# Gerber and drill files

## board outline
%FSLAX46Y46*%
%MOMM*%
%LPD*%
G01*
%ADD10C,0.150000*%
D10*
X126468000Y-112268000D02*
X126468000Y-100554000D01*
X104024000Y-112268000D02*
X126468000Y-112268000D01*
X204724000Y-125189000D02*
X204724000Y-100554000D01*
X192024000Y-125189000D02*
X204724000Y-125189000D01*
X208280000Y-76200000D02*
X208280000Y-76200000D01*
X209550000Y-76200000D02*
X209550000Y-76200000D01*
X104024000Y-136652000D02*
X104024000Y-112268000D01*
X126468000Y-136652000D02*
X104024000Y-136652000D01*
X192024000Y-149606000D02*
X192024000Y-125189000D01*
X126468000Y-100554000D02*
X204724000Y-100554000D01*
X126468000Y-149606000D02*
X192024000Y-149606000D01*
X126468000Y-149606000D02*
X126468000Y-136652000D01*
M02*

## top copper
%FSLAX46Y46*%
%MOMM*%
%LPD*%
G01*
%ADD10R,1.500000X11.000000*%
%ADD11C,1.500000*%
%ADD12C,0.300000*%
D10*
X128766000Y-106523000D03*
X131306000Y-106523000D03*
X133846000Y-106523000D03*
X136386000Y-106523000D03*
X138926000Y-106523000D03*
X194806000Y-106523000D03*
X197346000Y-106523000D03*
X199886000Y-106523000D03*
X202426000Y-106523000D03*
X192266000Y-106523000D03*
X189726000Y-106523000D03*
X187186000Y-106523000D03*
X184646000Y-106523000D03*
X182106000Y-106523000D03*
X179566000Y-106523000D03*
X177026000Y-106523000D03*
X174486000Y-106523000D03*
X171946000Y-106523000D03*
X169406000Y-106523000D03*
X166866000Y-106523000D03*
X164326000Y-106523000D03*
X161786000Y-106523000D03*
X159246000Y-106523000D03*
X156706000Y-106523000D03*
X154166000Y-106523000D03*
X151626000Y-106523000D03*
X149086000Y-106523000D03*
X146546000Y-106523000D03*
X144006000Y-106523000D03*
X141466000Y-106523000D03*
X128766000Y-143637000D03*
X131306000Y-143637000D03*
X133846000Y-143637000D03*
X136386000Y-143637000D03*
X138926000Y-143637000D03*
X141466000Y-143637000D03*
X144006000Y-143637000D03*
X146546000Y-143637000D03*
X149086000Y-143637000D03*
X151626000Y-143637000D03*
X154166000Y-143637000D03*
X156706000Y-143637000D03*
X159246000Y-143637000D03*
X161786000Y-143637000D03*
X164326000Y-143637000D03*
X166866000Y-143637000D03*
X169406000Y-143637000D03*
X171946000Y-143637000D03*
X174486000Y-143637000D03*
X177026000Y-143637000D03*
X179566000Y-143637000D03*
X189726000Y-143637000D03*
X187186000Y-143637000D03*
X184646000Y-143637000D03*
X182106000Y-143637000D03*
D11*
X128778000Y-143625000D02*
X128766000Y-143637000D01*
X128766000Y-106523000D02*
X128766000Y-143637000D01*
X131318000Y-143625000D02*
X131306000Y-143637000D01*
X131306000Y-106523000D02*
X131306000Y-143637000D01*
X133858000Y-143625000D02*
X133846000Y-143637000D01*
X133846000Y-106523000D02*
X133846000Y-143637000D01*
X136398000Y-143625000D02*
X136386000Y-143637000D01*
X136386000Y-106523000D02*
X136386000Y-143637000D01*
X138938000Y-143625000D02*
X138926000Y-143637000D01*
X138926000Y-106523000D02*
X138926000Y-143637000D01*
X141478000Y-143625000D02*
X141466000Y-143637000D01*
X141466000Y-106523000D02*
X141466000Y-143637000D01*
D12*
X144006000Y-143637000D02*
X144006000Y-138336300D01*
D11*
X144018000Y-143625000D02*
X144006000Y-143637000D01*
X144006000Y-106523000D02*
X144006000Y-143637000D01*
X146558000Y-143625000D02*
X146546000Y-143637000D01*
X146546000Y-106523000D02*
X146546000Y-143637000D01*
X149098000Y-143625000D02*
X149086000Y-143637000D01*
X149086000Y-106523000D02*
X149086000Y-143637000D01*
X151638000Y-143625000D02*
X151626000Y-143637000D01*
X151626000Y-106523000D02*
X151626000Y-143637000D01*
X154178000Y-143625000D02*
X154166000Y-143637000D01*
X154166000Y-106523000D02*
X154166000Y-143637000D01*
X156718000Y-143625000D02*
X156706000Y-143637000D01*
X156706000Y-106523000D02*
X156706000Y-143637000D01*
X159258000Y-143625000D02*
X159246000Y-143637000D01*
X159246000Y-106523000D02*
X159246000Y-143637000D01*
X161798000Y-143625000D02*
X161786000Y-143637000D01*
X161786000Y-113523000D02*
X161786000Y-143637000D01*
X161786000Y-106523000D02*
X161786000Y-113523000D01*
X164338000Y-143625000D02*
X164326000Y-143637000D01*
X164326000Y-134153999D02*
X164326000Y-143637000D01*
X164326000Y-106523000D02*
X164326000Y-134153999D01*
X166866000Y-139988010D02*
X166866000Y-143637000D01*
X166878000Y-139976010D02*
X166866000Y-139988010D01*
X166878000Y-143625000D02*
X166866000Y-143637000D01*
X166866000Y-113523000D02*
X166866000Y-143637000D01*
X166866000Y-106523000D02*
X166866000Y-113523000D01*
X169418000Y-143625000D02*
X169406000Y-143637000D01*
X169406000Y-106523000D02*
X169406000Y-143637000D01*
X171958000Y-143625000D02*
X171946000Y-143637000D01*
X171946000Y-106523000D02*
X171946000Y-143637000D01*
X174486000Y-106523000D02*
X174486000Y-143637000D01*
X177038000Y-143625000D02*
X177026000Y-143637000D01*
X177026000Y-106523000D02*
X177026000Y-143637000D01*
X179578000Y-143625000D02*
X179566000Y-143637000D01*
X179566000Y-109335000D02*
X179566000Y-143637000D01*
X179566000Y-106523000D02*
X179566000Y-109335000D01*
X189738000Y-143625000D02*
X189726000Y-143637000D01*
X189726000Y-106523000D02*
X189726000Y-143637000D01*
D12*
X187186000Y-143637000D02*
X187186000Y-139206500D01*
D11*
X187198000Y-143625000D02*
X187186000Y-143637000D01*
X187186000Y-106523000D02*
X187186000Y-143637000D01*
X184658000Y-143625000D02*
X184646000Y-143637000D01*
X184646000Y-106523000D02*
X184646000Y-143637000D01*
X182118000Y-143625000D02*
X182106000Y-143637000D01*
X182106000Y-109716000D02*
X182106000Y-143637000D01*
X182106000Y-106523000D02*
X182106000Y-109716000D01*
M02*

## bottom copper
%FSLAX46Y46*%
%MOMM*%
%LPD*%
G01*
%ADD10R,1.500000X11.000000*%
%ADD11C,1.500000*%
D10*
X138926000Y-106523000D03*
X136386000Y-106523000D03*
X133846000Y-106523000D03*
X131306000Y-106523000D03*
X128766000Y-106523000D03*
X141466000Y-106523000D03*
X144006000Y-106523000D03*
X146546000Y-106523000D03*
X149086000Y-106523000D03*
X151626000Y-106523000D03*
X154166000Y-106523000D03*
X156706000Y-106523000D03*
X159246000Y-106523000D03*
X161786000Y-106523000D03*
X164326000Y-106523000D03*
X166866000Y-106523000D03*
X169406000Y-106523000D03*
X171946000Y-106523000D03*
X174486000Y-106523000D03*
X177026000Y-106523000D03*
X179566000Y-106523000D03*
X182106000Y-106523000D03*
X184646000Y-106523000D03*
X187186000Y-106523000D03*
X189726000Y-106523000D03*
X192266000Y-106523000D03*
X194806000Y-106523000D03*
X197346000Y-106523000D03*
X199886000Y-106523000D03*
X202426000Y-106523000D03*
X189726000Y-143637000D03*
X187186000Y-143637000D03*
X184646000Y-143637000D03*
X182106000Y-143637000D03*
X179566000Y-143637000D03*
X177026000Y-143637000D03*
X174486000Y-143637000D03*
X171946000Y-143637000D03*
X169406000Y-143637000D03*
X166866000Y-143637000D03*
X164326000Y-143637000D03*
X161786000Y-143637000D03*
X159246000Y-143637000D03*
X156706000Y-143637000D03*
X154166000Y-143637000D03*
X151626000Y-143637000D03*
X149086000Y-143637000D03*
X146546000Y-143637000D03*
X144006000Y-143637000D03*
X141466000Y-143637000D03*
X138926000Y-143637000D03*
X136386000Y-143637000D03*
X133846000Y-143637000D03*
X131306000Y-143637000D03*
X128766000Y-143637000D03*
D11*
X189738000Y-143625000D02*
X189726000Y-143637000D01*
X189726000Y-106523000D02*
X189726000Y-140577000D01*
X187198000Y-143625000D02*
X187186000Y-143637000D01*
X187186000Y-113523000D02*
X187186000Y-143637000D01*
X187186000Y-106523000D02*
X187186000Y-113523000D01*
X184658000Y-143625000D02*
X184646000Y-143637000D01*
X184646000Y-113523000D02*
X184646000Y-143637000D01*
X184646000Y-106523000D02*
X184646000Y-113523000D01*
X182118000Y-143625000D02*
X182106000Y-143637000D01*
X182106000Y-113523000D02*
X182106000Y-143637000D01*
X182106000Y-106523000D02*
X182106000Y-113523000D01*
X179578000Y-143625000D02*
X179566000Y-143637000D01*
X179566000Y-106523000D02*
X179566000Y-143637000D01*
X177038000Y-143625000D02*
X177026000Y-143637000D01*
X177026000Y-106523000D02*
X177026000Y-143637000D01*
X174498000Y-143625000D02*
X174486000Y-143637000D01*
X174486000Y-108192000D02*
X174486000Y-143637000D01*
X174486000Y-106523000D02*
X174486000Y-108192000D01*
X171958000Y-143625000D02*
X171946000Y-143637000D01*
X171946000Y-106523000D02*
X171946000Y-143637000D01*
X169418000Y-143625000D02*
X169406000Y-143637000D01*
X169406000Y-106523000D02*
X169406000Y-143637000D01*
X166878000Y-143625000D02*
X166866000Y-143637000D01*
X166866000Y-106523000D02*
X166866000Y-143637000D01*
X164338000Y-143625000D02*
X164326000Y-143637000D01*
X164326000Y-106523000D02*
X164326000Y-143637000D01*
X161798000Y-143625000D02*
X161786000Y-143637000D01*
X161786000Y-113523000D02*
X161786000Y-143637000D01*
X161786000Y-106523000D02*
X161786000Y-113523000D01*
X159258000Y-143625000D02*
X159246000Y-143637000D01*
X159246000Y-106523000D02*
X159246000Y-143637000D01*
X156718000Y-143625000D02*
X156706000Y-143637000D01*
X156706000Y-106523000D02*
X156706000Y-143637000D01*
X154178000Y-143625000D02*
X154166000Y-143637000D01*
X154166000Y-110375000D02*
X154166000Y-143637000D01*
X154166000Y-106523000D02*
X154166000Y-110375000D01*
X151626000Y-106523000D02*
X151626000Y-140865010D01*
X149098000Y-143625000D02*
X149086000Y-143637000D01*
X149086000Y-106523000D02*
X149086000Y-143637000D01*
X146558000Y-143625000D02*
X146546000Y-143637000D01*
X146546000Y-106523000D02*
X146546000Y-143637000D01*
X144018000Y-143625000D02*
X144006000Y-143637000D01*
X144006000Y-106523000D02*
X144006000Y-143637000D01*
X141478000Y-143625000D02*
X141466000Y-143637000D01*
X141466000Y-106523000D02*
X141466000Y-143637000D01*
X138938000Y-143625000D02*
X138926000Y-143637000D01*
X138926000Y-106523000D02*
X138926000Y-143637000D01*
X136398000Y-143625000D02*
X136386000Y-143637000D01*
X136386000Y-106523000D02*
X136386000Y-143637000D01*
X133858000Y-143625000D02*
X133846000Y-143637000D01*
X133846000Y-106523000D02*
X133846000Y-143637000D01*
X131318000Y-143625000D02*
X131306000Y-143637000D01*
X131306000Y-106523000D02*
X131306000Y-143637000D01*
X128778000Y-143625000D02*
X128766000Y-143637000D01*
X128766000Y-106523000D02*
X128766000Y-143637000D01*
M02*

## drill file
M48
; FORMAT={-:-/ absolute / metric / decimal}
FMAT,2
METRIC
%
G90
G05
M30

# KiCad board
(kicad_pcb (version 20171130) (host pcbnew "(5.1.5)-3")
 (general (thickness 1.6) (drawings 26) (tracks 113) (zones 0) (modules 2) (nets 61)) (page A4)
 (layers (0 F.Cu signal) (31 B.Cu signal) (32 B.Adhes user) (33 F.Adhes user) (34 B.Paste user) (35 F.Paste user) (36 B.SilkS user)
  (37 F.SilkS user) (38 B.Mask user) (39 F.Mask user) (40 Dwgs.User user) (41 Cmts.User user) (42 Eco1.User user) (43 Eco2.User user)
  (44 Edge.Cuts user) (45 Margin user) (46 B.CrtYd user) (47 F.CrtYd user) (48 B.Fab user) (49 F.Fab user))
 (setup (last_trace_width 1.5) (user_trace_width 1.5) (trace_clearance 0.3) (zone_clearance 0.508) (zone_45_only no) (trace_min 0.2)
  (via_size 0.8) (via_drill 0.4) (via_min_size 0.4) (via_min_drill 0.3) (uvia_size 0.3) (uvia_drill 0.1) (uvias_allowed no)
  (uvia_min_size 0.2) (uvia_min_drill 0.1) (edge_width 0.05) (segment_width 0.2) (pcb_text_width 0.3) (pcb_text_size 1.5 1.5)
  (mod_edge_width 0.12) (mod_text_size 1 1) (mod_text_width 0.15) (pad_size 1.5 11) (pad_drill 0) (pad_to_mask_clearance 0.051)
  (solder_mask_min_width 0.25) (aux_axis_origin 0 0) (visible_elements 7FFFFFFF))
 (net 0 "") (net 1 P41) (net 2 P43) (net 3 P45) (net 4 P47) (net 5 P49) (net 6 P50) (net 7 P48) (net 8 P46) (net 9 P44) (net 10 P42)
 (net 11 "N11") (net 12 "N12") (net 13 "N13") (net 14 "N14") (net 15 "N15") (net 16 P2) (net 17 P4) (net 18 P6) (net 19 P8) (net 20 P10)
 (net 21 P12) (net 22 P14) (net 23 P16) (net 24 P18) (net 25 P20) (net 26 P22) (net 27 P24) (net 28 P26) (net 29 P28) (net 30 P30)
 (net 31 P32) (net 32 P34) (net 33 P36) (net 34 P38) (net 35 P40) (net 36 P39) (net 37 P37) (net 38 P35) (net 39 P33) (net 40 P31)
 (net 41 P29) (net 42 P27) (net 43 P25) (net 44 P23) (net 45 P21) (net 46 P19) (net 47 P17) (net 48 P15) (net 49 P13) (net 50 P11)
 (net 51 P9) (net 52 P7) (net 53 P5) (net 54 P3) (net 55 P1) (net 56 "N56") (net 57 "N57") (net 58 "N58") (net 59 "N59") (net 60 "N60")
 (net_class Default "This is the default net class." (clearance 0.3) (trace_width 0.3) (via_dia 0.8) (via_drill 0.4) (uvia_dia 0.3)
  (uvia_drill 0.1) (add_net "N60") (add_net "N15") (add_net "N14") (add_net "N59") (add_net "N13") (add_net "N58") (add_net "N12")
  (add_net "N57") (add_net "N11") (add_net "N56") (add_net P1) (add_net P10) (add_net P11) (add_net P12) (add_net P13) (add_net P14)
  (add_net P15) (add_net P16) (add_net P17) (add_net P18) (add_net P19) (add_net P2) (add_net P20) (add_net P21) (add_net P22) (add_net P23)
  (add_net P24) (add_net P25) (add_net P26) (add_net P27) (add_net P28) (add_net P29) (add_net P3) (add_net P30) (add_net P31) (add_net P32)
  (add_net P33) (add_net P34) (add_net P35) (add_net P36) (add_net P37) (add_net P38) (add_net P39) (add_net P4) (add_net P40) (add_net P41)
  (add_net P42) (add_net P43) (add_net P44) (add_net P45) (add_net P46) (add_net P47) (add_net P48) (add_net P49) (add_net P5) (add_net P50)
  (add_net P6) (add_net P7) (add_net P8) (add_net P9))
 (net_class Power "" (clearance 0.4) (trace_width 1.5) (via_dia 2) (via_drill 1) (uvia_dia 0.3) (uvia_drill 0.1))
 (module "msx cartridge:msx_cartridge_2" (layer F.Cu) (at 171.946 106.65)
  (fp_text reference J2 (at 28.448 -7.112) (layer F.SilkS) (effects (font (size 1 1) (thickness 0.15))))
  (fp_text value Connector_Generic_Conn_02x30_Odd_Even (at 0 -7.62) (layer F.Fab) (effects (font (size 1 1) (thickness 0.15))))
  (pad 51 connect rect (at -33.02 -0.127) (size 1.5 11) (layers B.Cu B.Mask) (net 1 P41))
  (pad 53 connect rect (at -35.56 -0.127) (size 1.5 11) (layers B.Cu B.Mask) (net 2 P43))
  (pad 55 connect rect (at -38.1 -0.127) (size 1.5 11) (layers B.Cu B.Mask) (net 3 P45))
  (pad 57 connect rect (at -40.64 -0.127) (size 1.5 11) (layers B.Cu B.Mask) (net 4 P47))
  (pad 59 connect rect (at -43.18 -0.127) (size 1.5 11) (layers B.Cu B.Mask) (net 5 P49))
  (pad 60 connect rect (at -43.18 -0.127) (size 1.5 11) (layers F.Cu F.Mask) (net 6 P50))
  (pad 58 connect rect (at -40.64 -0.127) (size 1.5 11) (layers F.Cu F.Mask) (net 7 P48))
  (pad 56 connect rect (at -38.1 -0.127) (size 1.5 11) (layers F.Cu F.Mask) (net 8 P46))
  (pad 54 connect rect (at -35.56 -0.127) (size 1.5 11) (layers F.Cu F.Mask) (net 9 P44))
  (pad 52 connect rect (at -33.02 -0.127) (size 1.5 11) (layers F.Cu F.Mask) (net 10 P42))
  (pad 8 connect rect (at 22.86 -0.127) (size 1.5 11) (layers F.Cu F.Mask) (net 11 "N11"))
  (pad 6 connect rect (at 25.4 -0.127) (size 1.5 11) (layers F.Cu F.Mask) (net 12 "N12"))
  (pad 4 connect rect (at 27.94 -0.127) (size 1.5 11) (layers F.Cu F.Mask) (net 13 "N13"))
  (pad 2 connect rect (at 30.48 -0.127) (size 1.5 11) (layers F.Cu F.Mask) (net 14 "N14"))
  (pad 10 connect rect (at 20.32 -0.127) (size 1.5 11) (layers F.Cu F.Mask) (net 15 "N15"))
  (pad 12 connect rect (at 17.78 -0.127) (size 1.5 11) (layers F.Cu F.Mask) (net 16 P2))
  (pad 14 connect rect (at 15.24 -0.127) (size 1.5 11) (layers F.Cu F.Mask) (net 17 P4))
  (pad 16 connect rect (at 12.7 -0.127) (size 1.5 11) (layers F.Cu F.Mask) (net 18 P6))
  (pad 18 connect rect (at 10.16 -0.127) (size 1.5 11) (layers F.Cu F.Mask) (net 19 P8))
  (pad 20 connect rect (at 7.62 -0.127) (size 1.5 11) (layers F.Cu F.Mask) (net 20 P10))
  (pad 22 connect rect (at 5.08 -0.127) (size 1.5 11) (layers F.Cu F.Mask) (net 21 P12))
  (pad 24 connect rect (at 2.54 -0.127) (size 1.5 11) (layers F.Cu F.Mask) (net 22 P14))
  (pad 26 connect rect (at 0 -0.127) (size 1.5 11) (layers F.Cu F.Mask) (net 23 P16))
  (pad 28 connect rect (at -2.54 -0.127) (size 1.5 11) (layers F.Cu F.Mask) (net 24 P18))
  (pad 30 connect rect (at -5.08 -0.127) (size 1.5 11) (layers F.Cu F.Mask) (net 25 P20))
  (pad 32 connect rect (at -7.62 -0.127) (size 1.5 11) (layers F.Cu F.Mask) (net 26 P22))
  (pad 34 connect rect (at -10.16 -0.127) (size 1.5 11) (layers F.Cu F.Mask) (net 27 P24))
  (pad 36 connect rect (at -12.7 -0.127) (size 1.5 11) (layers F.Cu F.Mask) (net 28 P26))
  (pad 38 connect rect (at -15.24 -0.127) (size 1.5 11) (layers F.Cu F.Mask) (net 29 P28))
  (pad 40 connect rect (at -17.78 -0.127) (size 1.5 11) (layers F.Cu F.Mask) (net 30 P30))
  (pad 42 connect rect (at -20.32 -0.127) (size 1.5 11) (layers F.Cu F.Mask) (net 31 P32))
  (pad 44 connect rect (at -22.86 -0.127) (size 1.5 11) (layers F.Cu F.Mask) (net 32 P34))
  (pad 46 connect rect (at -25.4 -0.127) (size 1.5 11) (layers F.Cu F.Mask) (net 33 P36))
  (pad 48 connect rect (at -27.94 -0.127) (size 1.5 11) (layers F.Cu F.Mask) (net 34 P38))
  (pad 50 connect rect (at -30.48 -0.127) (size 1.5 11) (layers F.Cu F.Mask) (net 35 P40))
  (pad 49 connect rect (at -30.48 -0.127) (size 1.5 11) (layers B.Cu B.Mask) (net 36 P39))
  (pad 47 connect rect (at -27.94 -0.127) (size 1.5 11) (layers B.Cu B.Mask) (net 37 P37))
  (pad 45 connect rect (at -25.4 -0.127) (size 1.5 11) (layers B.Cu B.Mask) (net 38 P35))
  (pad 43 connect rect (at -22.86 -0.127) (size 1.5 11) (layers B.Cu B.Mask) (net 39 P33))
  (pad 41 connect rect (at -20.32 -0.127) (size 1.5 11) (layers B.Cu B.Mask) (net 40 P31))
  (pad 39 connect rect (at -17.78 -0.127) (size 1.5 11) (layers B.Cu B.Mask) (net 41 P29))
  (pad 37 connect rect (at -15.24 -0.127) (size 1.5 11) (layers B.Cu B.Mask) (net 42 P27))
  (pad 35 connect rect (at -12.7 -0.127) (size 1.5 11) (layers B.Cu B.Mask) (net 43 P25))
  (pad 33 connect rect (at -10.16 -0.127) (size 1.5 11) (layers B.Cu B.Mask) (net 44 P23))
  (pad 31 connect rect (at -7.62 -0.127) (size 1.5 11) (layers B.Cu B.Mask) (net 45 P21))
  (pad 29 connect rect (at -5.08 -0.127) (size 1.5 11) (layers B.Cu B.Mask) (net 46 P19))
  (pad 27 connect rect (at -2.54 -0.127) (size 1.5 11) (layers B.Cu B.Mask) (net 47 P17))
  (pad 25 connect rect (at 0 -0.127) (size 1.5 11) (layers B.Cu B.Mask) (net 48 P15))
  (pad 23 connect rect (at 2.54 -0.127) (size 1.5 11) (layers B.Cu B.Mask) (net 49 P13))
  (pad 21 connect rect (at 5.08 -0.127) (size 1.5 11) (layers B.Cu B.Mask) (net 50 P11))
  (pad 19 connect rect (at 7.62 -0.127) (size 1.5 11) (layers B.Cu B.Mask) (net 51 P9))
  (pad 17 connect rect (at 10.16 -0.127) (size 1.5 11) (layers B.Cu B.Mask) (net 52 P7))
  (pad 15 connect rect (at 12.7 -0.127) (size 1.5 11) (layers B.Cu B.Mask) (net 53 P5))
  (pad 13 connect rect (at 15.24 -0.127) (size 1.5 11) (layers B.Cu B.Mask) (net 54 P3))
  (pad 11 connect rect (at 17.78 -0.127) (size 1.5 11) (layers B.Cu B.Mask) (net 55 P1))
  (pad 9 connect rect (at 20.32 -0.127) (size 1.5 11) (layers B.Cu B.Mask) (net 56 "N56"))
  (pad 7 connect rect (at 22.86 -0.127) (size 1.5 11) (layers B.Cu B.Mask) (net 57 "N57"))
  (pad 5 connect rect (at 25.4 -0.127) (size 1.5 11) (layers B.Cu B.Mask) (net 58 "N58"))
  (pad 3 connect rect (at 27.94 -0.127) (size 1.5 11) (layers B.Cu B.Mask) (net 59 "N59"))
  (pad 1 connect rect (at 30.48 -0.127) (size 1.5 11) (layers B.Cu B.Mask) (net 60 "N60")))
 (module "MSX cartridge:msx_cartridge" (layer F.Cu) (at 159.246 143.764)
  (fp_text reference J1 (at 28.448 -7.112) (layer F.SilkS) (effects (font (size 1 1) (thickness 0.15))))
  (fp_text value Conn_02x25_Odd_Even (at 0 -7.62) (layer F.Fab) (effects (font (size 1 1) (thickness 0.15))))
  (pad 1 connect rect (at 30.48 -0.127) (size 1.5 11) (layers B.Cu B.Mask) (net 55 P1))
  (pad 3 connect rect (at 27.94 -0.127) (size 1.5 11) (layers B.Cu B.Mask) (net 54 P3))
  (pad 5 connect rect (at 25.4 -0.127) (size 1.5 11) (layers B.Cu B.Mask) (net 53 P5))
  (pad 7 connect rect (at 22.86 -0.127) (size 1.5 11) (layers B.Cu B.Mask) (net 52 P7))
  (pad 9 connect rect (at 20.32 -0.127) (size 1.5 11) (layers B.Cu B.Mask) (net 51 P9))
  (pad 11 connect rect (at 17.78 -0.127) (size 1.5 11) (layers B.Cu B.Mask) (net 50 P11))
  (pad 13 connect rect (at 15.24 -0.127) (size 1.5 11) (layers B.Cu B.Mask) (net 49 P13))
  (pad 15 connect rect (at 12.7 -0.127) (size 1.5 11) (layers B.Cu B.Mask) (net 48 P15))
  (pad 17 connect rect (at 10.16 -0.127) (size 1.5 11) (layers B.Cu B.Mask) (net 47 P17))
  (pad 19 connect rect (at 7.62 -0.127) (size 1.5 11) (layers B.Cu B.Mask) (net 46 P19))
  (pad 21 connect rect (at 5.08 -0.127) (size 1.5 11) (layers B.Cu B.Mask) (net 45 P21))
  (pad 23 connect rect (at 2.54 -0.127) (size 1.5 11) (layers B.Cu B.Mask) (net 44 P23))
  (pad 25 connect rect (at 0 -0.127) (size 1.5 11) (layers B.Cu B.Mask) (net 43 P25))
  (pad 27 connect rect (at -2.54 -0.127) (size 1.5 11) (layers B.Cu B.Mask) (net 42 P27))
  (pad 29 connect rect (at -5.08 -0.127) (size 1.5 11) (layers B.Cu B.Mask) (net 41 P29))
  (pad 31 connect rect (at -7.62 -0.127) (size 1.5 11) (layers B.Cu B.Mask) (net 40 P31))
  (pad 33 connect rect (at -10.16 -0.127) (size 1.5 11) (layers B.Cu B.Mask) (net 39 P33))
  (pad 35 connect rect (at -12.7 -0.127) (size 1.5 11) (layers B.Cu B.Mask) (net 38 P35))
  (pad 37 connect rect (at -15.24 -0.127) (size 1.5 11) (layers B.Cu B.Mask) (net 37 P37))
  (pad 39 connect rect (at -17.78 -0.127) (size 1.5 11) (layers B.Cu B.Mask) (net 36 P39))
  (pad 41 connect rect (at -20.32 -0.127) (size 1.5 11) (layers B.Cu B.Mask) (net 1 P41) (zone_connect 2))
  (pad 43 connect rect (at -22.86 -0.127) (size 1.5 11) (layers B.Cu B.Mask) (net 2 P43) (zone_connect 2))
  (pad 45 connect rect (at -25.4 -0.127) (size 1.5 11) (layers B.Cu B.Mask) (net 3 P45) (zone_connect 2))
  (pad 47 connect rect (at -27.94 -0.127) (size 1.5 11) (layers B.Cu B.Mask) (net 4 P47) (zone_connect 2))
  (pad 49 connect rect (at -30.48 -0.127) (size 1.5 11) (layers B.Cu B.Mask) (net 5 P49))
  (pad 50 connect rect (at -30.48 -0.127) (size 1.5 11) (layers F.Cu F.Mask) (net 6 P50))
  (pad 48 connect rect (at -27.94 -0.127) (size 1.5 11) (layers F.Cu F.Mask) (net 7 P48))
  (pad 46 connect rect (at -25.4 -0.127) (size 1.5 11) (layers F.Cu F.Mask) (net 8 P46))
  (pad 44 connect rect (at -22.86 -0.127) (size 1.5 11) (layers F.Cu F.Mask) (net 9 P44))
  (pad 42 connect rect (at -20.32 -0.127) (size 1.5 11) (layers F.Cu F.Mask) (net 10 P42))
  (pad 40 connect rect (at -17.78 -0.127) (size 1.5 11) (layers F.Cu F.Mask) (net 35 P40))
  (pad 38 connect rect (at -15.24 -0.127) (size 1.5 11) (layers F.Cu F.Mask) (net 34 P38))
  (pad 36 connect rect (at -12.7 -0.127) (size 1.5 11) (layers F.Cu F.Mask) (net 33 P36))
  (pad 34 connect rect (at -10.16 -0.127) (size 1.5 11) (layers F.Cu F.Mask) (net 32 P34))
  (pad 32 connect rect (at -7.62 -0.127) (size 1.5 11) (layers F.Cu F.Mask) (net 31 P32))
  (pad 30 connect rect (at -5.08 -0.127) (size 1.5 11) (layers F.Cu F.Mask) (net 30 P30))
  (pad 28 connect rect (at -2.54 -0.127) (size 1.5 11) (layers F.Cu F.Mask) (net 29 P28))
  (pad 26 connect rect (at 0 -0.127) (size 1.5 11) (layers F.Cu F.Mask) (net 28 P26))
  (pad 24 connect rect (at 2.54 -0.127) (size 1.5 11) (layers F.Cu F.Mask) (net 27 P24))
  (pad 22 connect rect (at 5.08 -0.127) (size 1.5 11) (layers F.Cu F.Mask) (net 26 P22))
  (pad 20 connect rect (at 7.62 -0.127) (size 1.5 11) (layers F.Cu F.Mask) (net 25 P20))
  (pad 18 connect rect (at 10.16 -0.127) (size 1.5 11) (layers F.Cu F.Mask) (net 24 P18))
  (pad 16 connect rect (at 12.7 -0.127) (size 1.5 11) (layers F.Cu F.Mask) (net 23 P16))
  (pad 14 connect rect (at 15.24 -0.127) (size 1.5 11) (layers F.Cu F.Mask) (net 22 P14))
  (pad 12 connect rect (at 17.78 -0.127) (size 1.5 11) (layers F.Cu F.Mask) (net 21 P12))
  (pad 10 connect rect (at 20.32 -0.127) (size 1.5 11) (layers F.Cu F.Mask) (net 20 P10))
  (pad 2 connect rect (at 30.48 -0.127) (size 1.5 11) (layers F.Cu F.Mask) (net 16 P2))
  (pad 4 connect rect (at 27.94 -0.127) (size 1.5 11) (layers F.Cu F.Mask) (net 17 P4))
  (pad 6 connect rect (at 25.4 -0.127) (size 1.5 11) (layers F.Cu F.Mask) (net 18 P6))
  (pad 8 connect rect (at 22.86 -0.127) (size 1.5 11) (layers F.Cu F.Mask) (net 19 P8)))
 (gr_line (start 126.468 112.268) (end 126.468 100.554) (layer Edge.Cuts) (width 0.15))
 (gr_line (start 104.024 112.268) (end 126.468 112.268) (layer Edge.Cuts) (width 0.15))
 (gr_line (start 204.724 125.189) (end 204.724 100.554) (layer Edge.Cuts) (width 0.15))
 (gr_line (start 192.024 125.189) (end 204.724 125.189) (layer Edge.Cuts) (width 0.15))
 (gr_line (start 208.28 76.2) (end 208.28 76.2) (angle 90) (layer Edge.Cuts) (width 0.15))
 (gr_line (start 209.55 76.2) (end 209.55 76.2) (angle 90) (layer Edge.Cuts) (width 0.15))
 (gr_line (start 104.024 136.652) (end 104.024 112.268) (angle 90) (layer Edge.Cuts) (width 0.15))
 (gr_line (start 126.468 136.652) (end 104.024 136.652) (angle 90) (layer Edge.Cuts) (width 0.15))
 (gr_line (start 192.024 149.606) (end 192.024 125.189) (angle 90) (layer Edge.Cuts) (width 0.15))
 (gr_line (start 126.468 100.554) (end 204.724 100.554) (angle 90) (layer Edge.Cuts) (width 0.15))
 (gr_line (start 126.468 149.606) (end 192.024 149.606) (angle 90) (layer Edge.Cuts) (width 0.15))
 (gr_line (start 126.468 149.606) (end 126.468 136.652) (angle 90) (layer Edge.Cuts) (width 0.15))
 (segment (start 189.738 143.625) (end 189.726 143.637) (width 1.5) (layer B.Cu) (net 55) (status 30))
 (segment (start 189.726 106.523) (end 189.726 140.577) (width 1.5) (layer B.Cu) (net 55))
 (segment (start 187.198 143.625) (end 187.186 143.637) (width 1.5) (layer B.Cu) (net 54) (status 30))
 (segment (start 187.186 113.523) (end 187.186 143.637) (width 1.5) (layer B.Cu) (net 54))
 (segment (start 187.186 106.523) (end 187.186 113.523) (width 1.5) (layer B.Cu) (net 54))
 (segment (start 184.658 143.625) (end 184.646 143.637) (width 1.5) (layer B.Cu) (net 53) (status 30))
 (segment (start 184.646 113.523) (end 184.646 143.637) (width 1.5) (layer B.Cu) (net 53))
 (segment (start 184.646 106.523) (end 184.646 113.523) (width 1.5) (layer B.Cu) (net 53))
 (segment (start 182.118 143.625) (end 182.106 143.637) (width 1.5) (layer B.Cu) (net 52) (status 30))
 (segment (start 182.106 113.523) (end 182.106 143.637) (width 1.5) (layer B.Cu) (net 52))
 (segment (start 182.106 106.523) (end 182.106 113.523) (width 1.5) (layer B.Cu) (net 52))
 (segment (start 179.578 143.625) (end 179.566 143.637) (width 1.5) (layer B.Cu) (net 51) (status 30))
 (segment (start 179.566 106.523) (end 179.566 143.637) (width 1.5) (layer B.Cu) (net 51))
 (segment (start 177.038 143.625) (end 177.026 143.637) (width 1.5) (layer B.Cu) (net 50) (status 30))
 (segment (start 177.026 106.523) (end 177.026 143.637) (width 1.5) (layer B.Cu) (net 50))
 (segment (start 174.498 143.625) (end 174.486 143.637) (width 1.5) (layer B.Cu) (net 49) (status 30))
 (segment (start 174.486 108.192) (end 174.486 143.637) (width 1.5) (layer B.Cu) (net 49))
 (segment (start 174.486 106.523) (end 174.486 108.192) (width 1.5) (layer B.Cu) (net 49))
 (segment (start 171.958 143.625) (end 171.946 143.637) (width 1.5) (layer B.Cu) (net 48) (status 30))
 (segment (start 171.946 106.523) (end 171.946 143.637) (width 1.5) (layer B.Cu) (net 48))
 (segment (start 169.418 143.625) (end 169.406 143.637) (width 1.5) (layer B.Cu) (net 47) (status 30))
 (segment (start 169.406 106.523) (end 169.406 143.637) (width 1.5) (layer B.Cu) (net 47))
 (segment (start 166.878 143.625) (end 166.866 143.637) (width 1.5) (layer B.Cu) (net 46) (status 30))
 (segment (start 166.866 106.523) (end 166.866 143.637) (width 1.5) (layer B.Cu) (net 46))
 (segment (start 164.338 143.625) (end 164.326 143.637) (width 1.5) (layer B.Cu) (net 45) (status 30))
 (segment (start 164.326 106.523) (end 164.326 143.637) (width 1.5) (layer B.Cu) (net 45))
 (segment (start 161.798 143.625) (end 161.786 143.637) (width 1.5) (layer B.Cu) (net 44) (status 30))
 (segment (start 161.786 113.523) (end 161.786 143.637) (width 1.5) (layer B.Cu) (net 44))
 (segment (start 161.786 106.523) (end 161.786 113.523) (width 1.5) (layer B.Cu) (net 44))
 (segment (start 159.258 143.625) (end 159.246 143.637) (width 1.5) (layer B.Cu) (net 43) (status 30))
 (segment (start 159.246 106.523) (end 159.246 143.637) (width 1.5) (layer B.Cu) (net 43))
 (segment (start 156.718 143.625) (end 156.706 143.637) (width 1.5) (layer B.Cu) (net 42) (status 30))
 (segment (start 156.706 106.523) (end 156.706 143.637) (width 1.5) (layer B.Cu) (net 42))
 (segment (start 154.178 143.625) (end 154.166 143.637) (width 1.5) (layer B.Cu) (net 41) (status 30))
 (segment (start 154.166 110.375) (end 154.166 143.637) (width 1.5) (layer B.Cu) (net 41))
 (segment (start 154.166 106.523) (end 154.166 110.375) (width 1.5) (layer B.Cu) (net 41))
 (segment (start 151.626 106.523) (end 151.626 140.86501) (width 1.5) (layer B.Cu) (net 40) (status 30))
 (segment (start 149.098 143.625) (end 149.086 143.637) (width 1.5) (layer B.Cu) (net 39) (status 30))
 (segment (start 149.086 106.523) (end 149.086 143.637) (width 1.5) (layer B.Cu) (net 39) (status 30))
 (segment (start 146.558 143.625) (end 146.546 143.637) (width 1.5) (layer B.Cu) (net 38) (status 30))
 (segment (start 146.546 106.523) (end 146.546 143.637) (width 1.5) (layer B.Cu) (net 38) (status 30))
 (segment (start 144.018 143.625) (end 144.006 143.637) (width 1.5) (layer B.Cu) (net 37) (status 30))
 (segment (start 144.006 106.523) (end 144.006 143.637) (width 1.5) (layer B.Cu) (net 37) (status 30))
 (segment (start 141.478 143.625) (end 141.466 143.637) (width 1.5) (layer B.Cu) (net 36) (status 30))
 (segment (start 141.466 106.523) (end 141.466 143.637) (width 1.5) (layer B.Cu) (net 36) (status 30))
 (segment (start 138.938 143.625) (end 138.926 143.637) (width 1.5) (layer B.Cu) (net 1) (status 30))
 (segment (start 138.926 106.523) (end 138.926 143.637) (width 1.5) (layer B.Cu) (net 1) (status 30))
 (segment (start 136.398 143.625) (end 136.386 143.637) (width 1.5) (layer B.Cu) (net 2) (status 30))
 (segment (start 136.386 106.523) (end 136.386 143.637) (width 1.5) (layer B.Cu) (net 2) (status 30))
 (segment (start 133.858 143.625) (end 133.846 143.637) (width 1.5) (layer B.Cu) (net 3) (status 30))
 (segment (start 133.846 106.523) (end 133.846 143.637) (width 1.5) (layer B.Cu) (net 3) (status 30))
 (segment (start 131.318 143.625) (end 131.306 143.637) (width 1.5) (layer B.Cu) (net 4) (status 30))
 (segment (start 131.306 106.523) (end 131.306 143.637) (width 1.5) (layer B.Cu) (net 4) (status 30))
 (segment (start 128.778 143.625) (end 128.766 143.637) (width 1.5) (layer B.Cu) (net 5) (status 30))
 (segment (start 128.766 106.523) (end 128.766 143.637) (width 1.5) (layer B.Cu) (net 5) (status 30))
 (segment (start 128.778 143.625) (end 128.766 143.637) (width 1.5) (layer F.Cu) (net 6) (status 30))
 (segment (start 128.766 106.523) (end 128.766 143.637) (width 1.5) (layer F.Cu) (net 6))
 (segment (start 131.318 143.625) (end 131.306 143.637) (width 1.5) (layer F.Cu) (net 7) (status 30))
 (segment (start 131.306 106.523) (end 131.306 143.637) (width 1.5) (layer F.Cu) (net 7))
 (segment (start 133.858 143.625) (end 133.846 143.637) (width 1.5) (layer F.Cu) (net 8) (status 30))
 (segment (start 133.846 106.523) (end 133.846 143.637) (width 1.5) (layer F.Cu) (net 8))
 (segment (start 136.398 143.625) (end 136.386 143.637) (width 1.5) (layer F.Cu) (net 9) (status 30))
 (segment (start 136.386 106.523) (end 136.386 143.637) (width 1.5) (layer F.Cu) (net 9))
 (segment (start 138.938 143.625) (end 138.926 143.637) (width 1.5) (layer F.Cu) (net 10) (status 30))
 (segment (start 138.926 106.523) (end 138.926 143.637) (width 1.5) (layer F.Cu) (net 10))
 (segment (start 141.478 143.625) (end 141.466 143.637) (width 1.5) (layer F.Cu) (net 35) (status 30))
 (segment (start 141.466 106.523) (end 141.466 143.637) (width 1.5) (layer F.Cu) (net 35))
 (segment (start 144.006 143.637) (end 144.006 138.3363) (width 0.3) (layer F.Cu) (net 34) (status 30))
 (segment (start 144.018 143.625) (end 144.006 143.637) (width 1.5) (layer F.Cu) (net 34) (status 30))
 (segment (start 144.006 106.523) (end 144.006 143.637) (width 1.5) (layer F.Cu) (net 34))
 (segment (start 146.558 143.625) (end 146.546 143.637) (width 1.5) (layer F.Cu) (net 33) (status 30))
 (segment (start 146.546 106.523) (end 146.546 143.637) (width 1.5) (layer F.Cu) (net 33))
 (segment (start 149.098 143.625) (end 149.086 143.637) (width 1.5) (layer F.Cu) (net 32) (status 30))
 (segment (start 149.086 106.523) (end 149.086 143.637) (width 1.5) (layer F.Cu) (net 32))
 (segment (start 151.638 143.625) (end 151.626 143.637) (width 1.5) (layer F.Cu) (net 31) (status 30))
 (segment (start 151.626 106.523) (end 151.626 143.637) (width 1.5) (layer F.Cu) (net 31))
 (segment (start 154.178 143.625) (end 154.166 143.637) (width 1.5) (layer F.Cu) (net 30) (status 30))
 (segment (start 154.166 106.523) (end 154.166 143.637) (width 1.5) (layer F.Cu) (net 30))
 (segment (start 156.718 143.625) (end 156.706 143.637) (width 1.5) (layer F.Cu) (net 29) (status 30))
 (segment (start 156.706 106.523) (end 156.706 143.637) (width 1.5) (layer F.Cu) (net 29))
 (segment (start 159.258 143.625) (end 159.246 143.637) (width 1.5) (layer F.Cu) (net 28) (status 30))
 (segment (start 159.246 106.523) (end 159.246 143.637) (width 1.5) (layer F.Cu) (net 28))
 (segment (start 161.798 143.625) (end 161.786 143.637) (width 1.5) (layer F.Cu) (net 27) (status 30))
 (segment (start 161.786 113.523) (end 161.786 143.637) (width 1.5) (layer F.Cu) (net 27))
 (segment (start 161.786 106.523) (end 161.786 113.523) (width 1.5) (layer F.Cu) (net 27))
 (segment (start 164.338 143.625) (end 164.326 143.637) (width 1.5) (layer F.Cu) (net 26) (status 30))
 (segment (start 164.326 134.153999) (end 164.326 143.637) (width 1.5) (layer F.Cu) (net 26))
 (segment (start 164.326 106.523) (end 164.326 134.153999) (width 1.5) (layer F.Cu) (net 26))
 (segment (start 166.866 139.98801) (end 166.866 143.637) (width 1.5) (layer F.Cu) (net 25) (status 30))
 (segment (start 166.878 139.97601) (end 166.866 139.98801) (width 1.5) (layer F.Cu) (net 25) (status 30))
 (segment (start 166.878 143.625) (end 166.866 143.637) (width 1.5) (layer F.Cu) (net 25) (status 30))
 (segment (start 166.866 113.523) (end 166.866 143.637) (width 1.5) (layer F.Cu) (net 25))
 (segment (start 166.866 106.523) (end 166.866 113.523) (width 1.5) (layer F.Cu) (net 25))
 (segment (start 169.418 143.625) (end 169.406 143.637) (width 1.5) (layer F.Cu) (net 24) (status 30))
 (segment (start 169.406 106.523) (end 169.406 143.637) (width 1.5) (layer F.Cu) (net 24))
 (segment (start 171.958 143.625) (end 171.946 143.637) (width 1.5) (layer F.Cu) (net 23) (status 30))
 (segment (start 171.946 106.523) (end 171.946 143.637) (width 1.5) (layer F.Cu) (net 23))
 (segment (start 174.486 106.523) (end 174.486 143.637) (width 1.5) (layer F.Cu) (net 22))
 (segment (start 177.038 143.625) (end 177.026 143.637) (width 1.5) (layer F.Cu) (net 21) (status 30))
 (segment (start 177.026 106.523) (end 177.026 143.637) (width 1.5) (layer F.Cu) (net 21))
 (segment (start 179.578 143.625) (end 179.566 143.637) (width 1.5) (layer F.Cu) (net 20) (status 30))
 (segment (start 179.566 109.335) (end 179.566 143.637) (width 1.5) (layer F.Cu) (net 20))
 (segment (start 179.566 106.523) (end 179.566 109.335) (width 1.5) (layer F.Cu) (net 20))
 (segment (start 189.738 143.625) (end 189.726 143.637) (width 1.5) (layer F.Cu) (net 16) (status 30))
 (segment (start 189.726 106.523) (end 189.726 143.637) (width 1.5) (layer F.Cu) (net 16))
 (segment (start 187.186 143.637) (end 187.186 139.2065) (width 0.3) (layer F.Cu) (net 17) (status 30))
 (segment (start 187.198 143.625) (end 187.186 143.637) (width 1.5) (layer F.Cu) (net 17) (status 30))
 (segment (start 187.186 106.523) (end 187.186 143.637) (width 1.5) (layer F.Cu) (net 17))
 (segment (start 184.658 143.625) (end 184.646 143.637) (width 1.5) (layer F.Cu) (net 18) (status 30))
 (segment (start 184.646 106.523) (end 184.646 143.637) (width 1.5) (layer F.Cu) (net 18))
 (segment (start 182.118 143.625) (end 182.106 143.637) (width 1.5) (layer F.Cu) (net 19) (status 30))
 (segment (start 182.106 109.716) (end 182.106 143.637) (width 1.5) (layer F.Cu) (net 19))
 (segment (start 182.106 106.523) (end 182.106 109.716) (width 1.5) (layer F.Cu) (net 19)))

